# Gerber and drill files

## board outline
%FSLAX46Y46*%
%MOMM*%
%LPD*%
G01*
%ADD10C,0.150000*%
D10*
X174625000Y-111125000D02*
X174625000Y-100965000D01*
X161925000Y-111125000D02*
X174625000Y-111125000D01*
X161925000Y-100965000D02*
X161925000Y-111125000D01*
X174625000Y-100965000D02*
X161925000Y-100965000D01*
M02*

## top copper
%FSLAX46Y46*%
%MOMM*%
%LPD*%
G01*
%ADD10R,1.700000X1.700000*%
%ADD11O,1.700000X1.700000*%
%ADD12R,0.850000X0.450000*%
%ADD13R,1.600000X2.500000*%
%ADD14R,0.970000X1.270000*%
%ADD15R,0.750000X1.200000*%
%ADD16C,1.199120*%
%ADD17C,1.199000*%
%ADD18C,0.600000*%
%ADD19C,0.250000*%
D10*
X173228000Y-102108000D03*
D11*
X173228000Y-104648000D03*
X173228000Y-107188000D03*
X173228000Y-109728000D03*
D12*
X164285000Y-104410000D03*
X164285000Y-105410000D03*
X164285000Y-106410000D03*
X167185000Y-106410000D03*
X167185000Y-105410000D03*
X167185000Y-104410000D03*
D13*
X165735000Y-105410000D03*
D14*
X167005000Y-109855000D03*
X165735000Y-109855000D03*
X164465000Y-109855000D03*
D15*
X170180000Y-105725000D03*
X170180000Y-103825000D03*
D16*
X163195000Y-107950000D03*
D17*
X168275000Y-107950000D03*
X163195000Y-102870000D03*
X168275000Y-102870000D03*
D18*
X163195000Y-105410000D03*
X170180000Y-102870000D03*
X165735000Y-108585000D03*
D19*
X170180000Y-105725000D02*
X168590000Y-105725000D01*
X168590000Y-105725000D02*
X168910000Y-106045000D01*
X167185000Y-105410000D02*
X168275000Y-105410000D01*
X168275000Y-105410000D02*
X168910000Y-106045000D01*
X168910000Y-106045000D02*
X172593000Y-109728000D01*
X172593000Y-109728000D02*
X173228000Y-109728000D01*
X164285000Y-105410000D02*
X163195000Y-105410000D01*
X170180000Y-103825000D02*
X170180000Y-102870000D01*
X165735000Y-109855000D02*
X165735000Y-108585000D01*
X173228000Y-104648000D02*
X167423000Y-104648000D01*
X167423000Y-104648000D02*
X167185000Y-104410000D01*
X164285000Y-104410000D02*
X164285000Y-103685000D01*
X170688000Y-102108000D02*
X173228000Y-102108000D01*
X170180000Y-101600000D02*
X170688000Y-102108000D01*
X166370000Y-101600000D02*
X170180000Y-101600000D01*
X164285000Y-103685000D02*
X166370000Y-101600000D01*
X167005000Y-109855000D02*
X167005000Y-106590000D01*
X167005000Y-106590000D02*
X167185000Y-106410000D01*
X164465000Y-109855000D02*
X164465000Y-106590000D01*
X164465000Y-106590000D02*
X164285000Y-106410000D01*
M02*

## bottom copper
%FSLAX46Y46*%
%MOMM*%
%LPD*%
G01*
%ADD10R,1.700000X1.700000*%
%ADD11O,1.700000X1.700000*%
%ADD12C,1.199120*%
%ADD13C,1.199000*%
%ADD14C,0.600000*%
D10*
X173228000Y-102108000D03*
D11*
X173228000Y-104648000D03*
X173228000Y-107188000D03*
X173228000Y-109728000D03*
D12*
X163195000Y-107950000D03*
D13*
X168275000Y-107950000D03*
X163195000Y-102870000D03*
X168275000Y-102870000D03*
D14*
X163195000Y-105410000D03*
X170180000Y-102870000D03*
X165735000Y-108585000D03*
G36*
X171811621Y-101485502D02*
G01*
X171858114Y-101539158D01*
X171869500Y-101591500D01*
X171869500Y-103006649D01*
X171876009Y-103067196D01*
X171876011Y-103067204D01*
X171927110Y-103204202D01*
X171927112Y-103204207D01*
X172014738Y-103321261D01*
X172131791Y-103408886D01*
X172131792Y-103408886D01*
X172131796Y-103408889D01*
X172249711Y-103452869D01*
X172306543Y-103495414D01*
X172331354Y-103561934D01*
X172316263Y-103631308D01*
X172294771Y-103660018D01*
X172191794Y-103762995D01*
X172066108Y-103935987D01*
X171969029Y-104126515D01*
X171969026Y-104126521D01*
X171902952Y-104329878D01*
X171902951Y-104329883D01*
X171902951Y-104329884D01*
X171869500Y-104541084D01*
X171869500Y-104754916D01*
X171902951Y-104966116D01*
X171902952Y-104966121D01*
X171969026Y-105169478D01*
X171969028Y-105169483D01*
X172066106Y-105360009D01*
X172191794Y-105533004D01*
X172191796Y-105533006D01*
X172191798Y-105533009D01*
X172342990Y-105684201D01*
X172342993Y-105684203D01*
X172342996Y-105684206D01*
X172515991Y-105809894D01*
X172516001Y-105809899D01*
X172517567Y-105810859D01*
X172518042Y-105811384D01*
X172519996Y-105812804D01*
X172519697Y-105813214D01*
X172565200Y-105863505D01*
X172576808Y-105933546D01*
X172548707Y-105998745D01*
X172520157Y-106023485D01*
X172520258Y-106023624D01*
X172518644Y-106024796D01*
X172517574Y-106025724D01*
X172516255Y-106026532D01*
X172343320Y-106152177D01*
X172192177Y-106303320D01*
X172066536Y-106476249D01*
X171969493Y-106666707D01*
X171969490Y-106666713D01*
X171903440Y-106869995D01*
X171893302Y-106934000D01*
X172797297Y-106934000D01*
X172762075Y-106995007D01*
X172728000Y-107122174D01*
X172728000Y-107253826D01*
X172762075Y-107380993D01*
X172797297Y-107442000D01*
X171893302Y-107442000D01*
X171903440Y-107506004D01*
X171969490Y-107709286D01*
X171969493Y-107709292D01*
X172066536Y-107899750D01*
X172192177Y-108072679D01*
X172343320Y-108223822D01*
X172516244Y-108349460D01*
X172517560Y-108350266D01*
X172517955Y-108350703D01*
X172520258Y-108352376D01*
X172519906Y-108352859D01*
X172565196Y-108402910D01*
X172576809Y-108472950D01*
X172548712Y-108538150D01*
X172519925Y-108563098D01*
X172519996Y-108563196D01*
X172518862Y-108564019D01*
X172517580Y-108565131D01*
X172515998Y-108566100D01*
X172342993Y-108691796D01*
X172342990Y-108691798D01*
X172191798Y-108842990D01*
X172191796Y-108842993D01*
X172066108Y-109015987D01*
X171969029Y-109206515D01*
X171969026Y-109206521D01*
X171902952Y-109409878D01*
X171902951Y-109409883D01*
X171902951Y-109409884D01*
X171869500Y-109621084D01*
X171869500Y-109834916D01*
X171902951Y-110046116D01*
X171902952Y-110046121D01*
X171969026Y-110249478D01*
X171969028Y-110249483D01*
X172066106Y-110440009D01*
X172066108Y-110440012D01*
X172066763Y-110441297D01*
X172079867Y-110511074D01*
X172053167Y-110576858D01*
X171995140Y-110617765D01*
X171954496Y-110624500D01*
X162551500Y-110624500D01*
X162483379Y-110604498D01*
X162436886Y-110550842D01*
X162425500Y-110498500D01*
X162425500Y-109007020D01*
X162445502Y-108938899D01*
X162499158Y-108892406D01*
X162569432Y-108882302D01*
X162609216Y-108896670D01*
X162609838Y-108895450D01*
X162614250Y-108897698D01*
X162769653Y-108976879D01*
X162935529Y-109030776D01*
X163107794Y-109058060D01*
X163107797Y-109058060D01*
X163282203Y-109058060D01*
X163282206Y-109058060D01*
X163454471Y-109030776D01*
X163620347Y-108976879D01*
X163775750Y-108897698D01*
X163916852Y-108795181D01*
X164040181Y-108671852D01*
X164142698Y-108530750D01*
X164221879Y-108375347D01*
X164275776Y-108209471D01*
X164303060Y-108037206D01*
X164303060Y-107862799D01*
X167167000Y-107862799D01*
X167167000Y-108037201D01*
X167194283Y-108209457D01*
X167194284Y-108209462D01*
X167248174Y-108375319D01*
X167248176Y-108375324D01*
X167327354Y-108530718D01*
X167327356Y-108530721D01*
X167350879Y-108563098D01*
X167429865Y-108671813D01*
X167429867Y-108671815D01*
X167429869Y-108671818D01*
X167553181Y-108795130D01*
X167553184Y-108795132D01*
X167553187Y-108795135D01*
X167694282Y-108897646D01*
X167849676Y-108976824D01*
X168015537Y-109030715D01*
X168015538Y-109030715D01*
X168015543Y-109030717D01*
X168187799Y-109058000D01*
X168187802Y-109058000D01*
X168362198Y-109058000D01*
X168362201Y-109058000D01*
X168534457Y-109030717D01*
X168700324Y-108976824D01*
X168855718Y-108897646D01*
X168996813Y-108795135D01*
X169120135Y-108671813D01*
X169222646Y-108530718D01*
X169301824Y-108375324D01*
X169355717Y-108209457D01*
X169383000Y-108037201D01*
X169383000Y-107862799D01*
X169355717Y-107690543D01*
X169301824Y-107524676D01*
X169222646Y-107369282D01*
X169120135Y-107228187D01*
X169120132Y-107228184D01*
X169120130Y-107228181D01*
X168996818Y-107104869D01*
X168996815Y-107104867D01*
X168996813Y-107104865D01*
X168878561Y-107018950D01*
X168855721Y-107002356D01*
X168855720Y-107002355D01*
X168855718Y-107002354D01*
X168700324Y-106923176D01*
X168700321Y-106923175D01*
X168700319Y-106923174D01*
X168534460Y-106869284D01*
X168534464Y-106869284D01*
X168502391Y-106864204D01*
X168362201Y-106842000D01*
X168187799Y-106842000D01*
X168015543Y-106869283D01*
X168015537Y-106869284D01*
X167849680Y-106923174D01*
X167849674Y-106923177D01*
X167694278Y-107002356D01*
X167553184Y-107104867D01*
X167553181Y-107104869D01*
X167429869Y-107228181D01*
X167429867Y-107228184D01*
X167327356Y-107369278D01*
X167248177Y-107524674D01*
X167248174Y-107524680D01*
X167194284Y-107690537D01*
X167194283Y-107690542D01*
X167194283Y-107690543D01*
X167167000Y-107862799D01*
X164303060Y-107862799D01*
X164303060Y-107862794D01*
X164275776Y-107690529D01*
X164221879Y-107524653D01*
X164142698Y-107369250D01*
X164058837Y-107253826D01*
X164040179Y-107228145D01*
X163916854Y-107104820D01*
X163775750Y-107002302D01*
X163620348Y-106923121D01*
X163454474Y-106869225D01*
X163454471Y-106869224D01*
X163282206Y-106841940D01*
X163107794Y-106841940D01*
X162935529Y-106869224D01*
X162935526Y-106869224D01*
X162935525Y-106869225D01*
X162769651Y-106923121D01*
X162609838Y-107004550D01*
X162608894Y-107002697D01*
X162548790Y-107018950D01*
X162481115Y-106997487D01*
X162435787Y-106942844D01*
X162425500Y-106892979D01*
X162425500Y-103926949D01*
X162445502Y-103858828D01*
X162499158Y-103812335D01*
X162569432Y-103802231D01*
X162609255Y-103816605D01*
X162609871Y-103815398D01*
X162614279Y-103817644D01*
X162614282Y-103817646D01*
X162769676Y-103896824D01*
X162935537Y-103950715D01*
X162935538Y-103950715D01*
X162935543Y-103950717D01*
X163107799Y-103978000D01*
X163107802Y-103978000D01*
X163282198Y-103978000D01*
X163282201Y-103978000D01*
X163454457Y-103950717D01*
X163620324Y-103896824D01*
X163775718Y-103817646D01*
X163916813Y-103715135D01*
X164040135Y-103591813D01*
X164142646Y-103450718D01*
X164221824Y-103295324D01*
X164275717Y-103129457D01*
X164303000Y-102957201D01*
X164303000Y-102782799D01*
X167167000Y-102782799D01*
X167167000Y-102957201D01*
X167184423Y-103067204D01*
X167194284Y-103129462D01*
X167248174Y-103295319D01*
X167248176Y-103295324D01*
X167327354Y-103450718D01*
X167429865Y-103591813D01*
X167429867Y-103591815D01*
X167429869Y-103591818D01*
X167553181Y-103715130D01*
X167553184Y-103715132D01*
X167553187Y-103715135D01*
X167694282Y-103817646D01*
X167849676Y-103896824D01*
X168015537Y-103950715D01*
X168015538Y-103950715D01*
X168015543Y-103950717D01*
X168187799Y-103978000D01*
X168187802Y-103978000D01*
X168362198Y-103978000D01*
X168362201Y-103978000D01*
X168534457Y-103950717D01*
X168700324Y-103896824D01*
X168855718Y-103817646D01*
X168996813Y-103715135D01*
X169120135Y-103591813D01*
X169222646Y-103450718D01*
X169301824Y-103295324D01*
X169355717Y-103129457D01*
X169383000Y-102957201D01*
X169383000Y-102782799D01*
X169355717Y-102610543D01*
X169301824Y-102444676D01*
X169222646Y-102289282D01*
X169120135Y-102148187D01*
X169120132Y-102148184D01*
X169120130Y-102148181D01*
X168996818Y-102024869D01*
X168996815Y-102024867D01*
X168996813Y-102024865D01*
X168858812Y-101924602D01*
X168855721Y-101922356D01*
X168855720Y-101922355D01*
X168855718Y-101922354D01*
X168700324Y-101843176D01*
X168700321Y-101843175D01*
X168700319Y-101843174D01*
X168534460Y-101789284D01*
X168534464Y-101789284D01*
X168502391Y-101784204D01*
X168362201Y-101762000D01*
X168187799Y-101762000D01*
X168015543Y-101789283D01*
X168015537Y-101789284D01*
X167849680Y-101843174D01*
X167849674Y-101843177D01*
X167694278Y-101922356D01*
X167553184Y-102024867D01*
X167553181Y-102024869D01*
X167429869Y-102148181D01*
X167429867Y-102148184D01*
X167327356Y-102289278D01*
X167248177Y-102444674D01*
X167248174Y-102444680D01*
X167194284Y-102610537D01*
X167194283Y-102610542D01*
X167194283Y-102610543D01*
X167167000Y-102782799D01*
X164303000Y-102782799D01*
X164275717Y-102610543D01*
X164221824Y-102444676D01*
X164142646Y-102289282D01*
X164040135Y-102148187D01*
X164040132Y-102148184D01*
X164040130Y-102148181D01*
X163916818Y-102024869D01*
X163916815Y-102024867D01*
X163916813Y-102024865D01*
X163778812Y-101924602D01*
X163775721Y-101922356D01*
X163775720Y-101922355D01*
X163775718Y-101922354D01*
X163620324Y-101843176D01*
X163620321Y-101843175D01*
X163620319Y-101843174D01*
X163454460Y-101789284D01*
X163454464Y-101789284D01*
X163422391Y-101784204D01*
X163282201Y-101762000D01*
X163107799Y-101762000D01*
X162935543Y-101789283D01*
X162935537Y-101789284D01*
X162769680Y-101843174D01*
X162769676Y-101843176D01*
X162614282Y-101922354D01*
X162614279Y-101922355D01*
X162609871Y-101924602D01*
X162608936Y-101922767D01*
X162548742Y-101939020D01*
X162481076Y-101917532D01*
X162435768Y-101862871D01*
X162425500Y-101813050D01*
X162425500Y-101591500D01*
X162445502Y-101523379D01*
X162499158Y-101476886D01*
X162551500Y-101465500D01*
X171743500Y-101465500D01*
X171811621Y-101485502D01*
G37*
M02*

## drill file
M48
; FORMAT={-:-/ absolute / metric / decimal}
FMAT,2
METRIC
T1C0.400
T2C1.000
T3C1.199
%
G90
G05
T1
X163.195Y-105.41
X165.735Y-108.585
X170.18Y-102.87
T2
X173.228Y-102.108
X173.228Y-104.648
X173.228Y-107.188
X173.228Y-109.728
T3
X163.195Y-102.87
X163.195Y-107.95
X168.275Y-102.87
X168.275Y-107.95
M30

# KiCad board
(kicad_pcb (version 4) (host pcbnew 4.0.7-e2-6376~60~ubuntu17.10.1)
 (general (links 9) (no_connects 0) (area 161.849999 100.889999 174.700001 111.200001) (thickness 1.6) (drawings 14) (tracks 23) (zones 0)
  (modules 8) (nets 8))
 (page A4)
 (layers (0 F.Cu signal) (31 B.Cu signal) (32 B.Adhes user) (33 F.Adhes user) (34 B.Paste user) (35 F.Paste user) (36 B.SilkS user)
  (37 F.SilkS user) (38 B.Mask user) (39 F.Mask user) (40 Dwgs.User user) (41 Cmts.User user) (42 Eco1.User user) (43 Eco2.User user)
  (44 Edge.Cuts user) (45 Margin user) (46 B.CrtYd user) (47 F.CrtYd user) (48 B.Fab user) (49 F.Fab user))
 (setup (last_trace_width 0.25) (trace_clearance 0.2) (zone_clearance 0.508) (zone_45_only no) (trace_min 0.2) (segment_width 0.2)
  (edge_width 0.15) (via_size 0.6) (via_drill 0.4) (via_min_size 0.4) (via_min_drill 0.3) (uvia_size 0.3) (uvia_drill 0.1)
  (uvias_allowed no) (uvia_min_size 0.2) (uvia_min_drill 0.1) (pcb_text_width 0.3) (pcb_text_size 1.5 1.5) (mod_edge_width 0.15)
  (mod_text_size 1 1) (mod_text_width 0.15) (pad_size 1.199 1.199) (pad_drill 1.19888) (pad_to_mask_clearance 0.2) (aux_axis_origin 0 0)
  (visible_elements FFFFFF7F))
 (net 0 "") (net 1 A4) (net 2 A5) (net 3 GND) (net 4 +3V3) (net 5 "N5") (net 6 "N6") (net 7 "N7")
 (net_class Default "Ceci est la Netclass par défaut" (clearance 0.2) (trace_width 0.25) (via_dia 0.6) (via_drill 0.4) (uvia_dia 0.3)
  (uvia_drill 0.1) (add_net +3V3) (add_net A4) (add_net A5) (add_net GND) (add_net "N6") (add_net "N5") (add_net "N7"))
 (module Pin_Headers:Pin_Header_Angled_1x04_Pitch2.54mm (layer B.Cu) (at 173.228 102.108 180)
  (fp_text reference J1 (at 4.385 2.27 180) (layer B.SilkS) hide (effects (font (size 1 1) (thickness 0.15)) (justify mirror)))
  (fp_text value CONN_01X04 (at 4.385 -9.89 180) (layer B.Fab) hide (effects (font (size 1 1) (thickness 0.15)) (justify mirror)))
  (pad 1 thru_hole rect (at 0 0 180) (size 1.7 1.7) (drill 1) (layers *.Cu *.Mask) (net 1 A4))
  (pad 2 thru_hole oval (at 0 -2.54 180) (size 1.7 1.7) (drill 1) (layers *.Cu *.Mask) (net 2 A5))
  (pad 3 thru_hole oval (at 0 -5.08 180) (size 1.7 1.7) (drill 1) (layers *.Cu *.Mask) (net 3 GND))
  (pad 4 thru_hole oval (at 0 -7.62 180) (size 1.7 1.7) (drill 1) (layers *.Cu *.Mask) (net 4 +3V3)))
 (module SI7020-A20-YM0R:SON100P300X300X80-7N (layer F.Cu) (at 165.735 105.41)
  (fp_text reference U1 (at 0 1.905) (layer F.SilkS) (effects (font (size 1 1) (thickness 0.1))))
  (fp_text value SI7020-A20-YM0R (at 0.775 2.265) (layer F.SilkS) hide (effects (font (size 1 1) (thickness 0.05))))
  (pad 1 smd rect (at -1.45 -1) (size 0.85 0.45) (layers F.Cu F.Paste F.Mask) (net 1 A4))
  (pad 2 smd rect (at -1.45 0) (size 0.85 0.45) (layers F.Cu F.Paste F.Mask) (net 3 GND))
  (pad 3 smd rect (at -1.45 1) (size 0.85 0.45) (layers F.Cu F.Paste F.Mask) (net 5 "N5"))
  (pad 4 smd rect (at 1.45 1 180) (size 0.85 0.45) (layers F.Cu F.Paste F.Mask) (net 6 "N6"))
  (pad 5 smd rect (at 1.45 0 180) (size 0.85 0.45) (layers F.Cu F.Paste F.Mask) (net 4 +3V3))
  (pad 6 smd rect (at 1.45 -1 180) (size 0.85 0.45) (layers F.Cu F.Paste F.Mask) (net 2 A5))
  (pad 7 smd rect (at 0 0) (size 1.6 2.5) (layers F.Cu F.Paste F.Mask) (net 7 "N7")))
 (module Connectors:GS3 (layer F.Cu) (at 165.735 109.855 270)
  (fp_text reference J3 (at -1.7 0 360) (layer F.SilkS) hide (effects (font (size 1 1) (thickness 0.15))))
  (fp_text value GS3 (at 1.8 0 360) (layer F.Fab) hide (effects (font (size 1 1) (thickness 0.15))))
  (pad 1 smd rect (at 0 -1.27 270) (size 1.27 0.97) (layers F.Cu F.Paste F.Mask) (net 6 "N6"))
  (pad 2 smd rect (at 0 0 270) (size 1.27 0.97) (layers F.Cu F.Paste F.Mask) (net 3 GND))
  (pad 3 smd rect (at 0 1.27 270) (size 1.27 0.97) (layers F.Cu F.Paste F.Mask) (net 5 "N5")))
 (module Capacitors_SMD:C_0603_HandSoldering (layer F.Cu) (at 170.18 104.775 90)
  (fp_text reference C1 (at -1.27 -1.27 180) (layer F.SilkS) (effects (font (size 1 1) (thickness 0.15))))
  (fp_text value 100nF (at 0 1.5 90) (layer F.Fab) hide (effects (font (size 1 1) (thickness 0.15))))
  (pad 1 smd rect (at -0.95 0 90) (size 1.2 0.75) (layers F.Cu F.Paste F.Mask) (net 4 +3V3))
  (pad 2 smd rect (at 0.95 0 90) (size 1.2 0.75) (layers F.Cu F.Paste F.Mask) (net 3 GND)))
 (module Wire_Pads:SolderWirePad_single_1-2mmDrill (layer F.Cu) (at 163.195 107.95)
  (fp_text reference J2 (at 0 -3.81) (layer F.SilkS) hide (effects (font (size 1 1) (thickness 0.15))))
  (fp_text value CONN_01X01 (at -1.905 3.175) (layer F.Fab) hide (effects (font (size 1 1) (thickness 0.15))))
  (pad "" np_thru_hole circle (at 0 0) (size 1.19912 1.19912) (drill 1.19888) (layers *.Cu *.Mask)))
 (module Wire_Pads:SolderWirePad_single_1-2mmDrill (layer F.Cu) (at 168.275 107.95)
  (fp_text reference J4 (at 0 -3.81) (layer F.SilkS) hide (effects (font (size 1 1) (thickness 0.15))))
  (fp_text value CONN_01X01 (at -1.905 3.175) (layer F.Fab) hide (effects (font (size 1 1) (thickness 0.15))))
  (pad "" np_thru_hole circle (at 0 0) (size 1.199 1.199) (drill 1.19888) (layers *.Cu *.Mask)))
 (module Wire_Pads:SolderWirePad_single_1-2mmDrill (layer F.Cu) (at 163.195 102.87)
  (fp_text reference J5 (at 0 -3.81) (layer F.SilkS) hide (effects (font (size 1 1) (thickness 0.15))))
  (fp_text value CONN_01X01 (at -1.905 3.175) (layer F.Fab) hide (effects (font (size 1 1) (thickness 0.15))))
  (pad "" np_thru_hole circle (at 0 0) (size 1.199 1.199) (drill 1.19888) (layers *.Cu *.Mask)))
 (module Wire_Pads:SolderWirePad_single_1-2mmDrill (layer F.Cu) (at 168.275 102.87)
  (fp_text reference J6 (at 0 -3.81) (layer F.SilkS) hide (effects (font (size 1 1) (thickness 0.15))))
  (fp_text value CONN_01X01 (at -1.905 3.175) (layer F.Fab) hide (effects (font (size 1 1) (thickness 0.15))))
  (pad "" np_thru_hole circle (at 0 0) (size 1.199 1.199) (drill 1.19888) (layers *.Cu *.Mask)))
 (gr_line (start 174.625 111.125) (end 174.625 100.965) (angle 90) (layer Edge.Cuts) (width 0.15))
 (gr_line (start 161.925 111.125) (end 174.625 111.125) (angle 90) (layer Edge.Cuts) (width 0.15))
 (gr_line (start 161.925 100.965) (end 161.925 111.125) (angle 90) (layer Edge.Cuts) (width 0.15))
 (gr_line (start 174.625 100.965) (end 161.925 100.965) (angle 90) (layer Edge.Cuts) (width 0.15))
 (segment (start 170.18 105.725) (end 168.59 105.725) (width 0.25) (layer F.Cu) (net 4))
 (segment (start 168.59 105.725) (end 168.91 106.045) (width 0.25) (layer F.Cu) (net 4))
 (segment (start 167.185 105.41) (end 168.275 105.41) (width 0.25) (layer F.Cu) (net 4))
 (segment (start 168.275 105.41) (end 168.91 106.045) (width 0.25) (layer F.Cu) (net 4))
 (segment (start 168.91 106.045) (end 172.593 109.728) (width 0.25) (layer F.Cu) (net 4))
 (segment (start 172.593 109.728) (end 173.228 109.728) (width 0.25) (layer F.Cu) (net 4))
 (segment (start 164.285 105.41) (end 163.195 105.41) (width 0.25) (layer F.Cu) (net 3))
 (via (at 163.195 105.41) (size 0.6) (drill 0.4) (layers F.Cu B.Cu) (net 3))
 (segment (start 170.18 103.825) (end 170.18 102.87) (width 0.25) (layer F.Cu) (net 3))
 (via (at 170.18 102.87) (size 0.6) (drill 0.4) (layers F.Cu B.Cu) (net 3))
 (segment (start 165.735 109.855) (end 165.735 108.585) (width 0.25) (layer F.Cu) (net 3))
 (via (at 165.735 108.585) (size 0.6) (drill 0.4) (layers F.Cu B.Cu) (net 3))
 (segment (start 173.228 104.648) (end 167.423 104.648) (width 0.25) (layer F.Cu) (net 2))
 (segment (start 167.423 104.648) (end 167.185 104.41) (width 0.25) (layer F.Cu) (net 2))
 (segment (start 164.285 104.41) (end 164.285 103.685) (width 0.25) (layer F.Cu) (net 1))
 (segment (start 170.688 102.108) (end 173.228 102.108) (width 0.25) (layer F.Cu) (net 1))
 (segment (start 170.18 101.6) (end 170.688 102.108) (width 0.25) (layer F.Cu) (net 1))
 (segment (start 166.37 101.6) (end 170.18 101.6) (width 0.25) (layer F.Cu) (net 1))
 (segment (start 164.285 103.685) (end 166.37 101.6) (width 0.25) (layer F.Cu) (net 1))
 (segment (start 167.005 109.855) (end 167.005 106.59) (width 0.25) (layer F.Cu) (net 6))
 (segment (start 167.005 106.59) (end 167.185 106.41) (width 0.25) (layer F.Cu) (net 6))
 (segment (start 164.465 109.855) (end 164.465 106.59) (width 0.25) (layer F.Cu) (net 5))
 (segment (start 164.465 106.59) (end 164.285 106.41) (width 0.25) (layer F.Cu) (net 5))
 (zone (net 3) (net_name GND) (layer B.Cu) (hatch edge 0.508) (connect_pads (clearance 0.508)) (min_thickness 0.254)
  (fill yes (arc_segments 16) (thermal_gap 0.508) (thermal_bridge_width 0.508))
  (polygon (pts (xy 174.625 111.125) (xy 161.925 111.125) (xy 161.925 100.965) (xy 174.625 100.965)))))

